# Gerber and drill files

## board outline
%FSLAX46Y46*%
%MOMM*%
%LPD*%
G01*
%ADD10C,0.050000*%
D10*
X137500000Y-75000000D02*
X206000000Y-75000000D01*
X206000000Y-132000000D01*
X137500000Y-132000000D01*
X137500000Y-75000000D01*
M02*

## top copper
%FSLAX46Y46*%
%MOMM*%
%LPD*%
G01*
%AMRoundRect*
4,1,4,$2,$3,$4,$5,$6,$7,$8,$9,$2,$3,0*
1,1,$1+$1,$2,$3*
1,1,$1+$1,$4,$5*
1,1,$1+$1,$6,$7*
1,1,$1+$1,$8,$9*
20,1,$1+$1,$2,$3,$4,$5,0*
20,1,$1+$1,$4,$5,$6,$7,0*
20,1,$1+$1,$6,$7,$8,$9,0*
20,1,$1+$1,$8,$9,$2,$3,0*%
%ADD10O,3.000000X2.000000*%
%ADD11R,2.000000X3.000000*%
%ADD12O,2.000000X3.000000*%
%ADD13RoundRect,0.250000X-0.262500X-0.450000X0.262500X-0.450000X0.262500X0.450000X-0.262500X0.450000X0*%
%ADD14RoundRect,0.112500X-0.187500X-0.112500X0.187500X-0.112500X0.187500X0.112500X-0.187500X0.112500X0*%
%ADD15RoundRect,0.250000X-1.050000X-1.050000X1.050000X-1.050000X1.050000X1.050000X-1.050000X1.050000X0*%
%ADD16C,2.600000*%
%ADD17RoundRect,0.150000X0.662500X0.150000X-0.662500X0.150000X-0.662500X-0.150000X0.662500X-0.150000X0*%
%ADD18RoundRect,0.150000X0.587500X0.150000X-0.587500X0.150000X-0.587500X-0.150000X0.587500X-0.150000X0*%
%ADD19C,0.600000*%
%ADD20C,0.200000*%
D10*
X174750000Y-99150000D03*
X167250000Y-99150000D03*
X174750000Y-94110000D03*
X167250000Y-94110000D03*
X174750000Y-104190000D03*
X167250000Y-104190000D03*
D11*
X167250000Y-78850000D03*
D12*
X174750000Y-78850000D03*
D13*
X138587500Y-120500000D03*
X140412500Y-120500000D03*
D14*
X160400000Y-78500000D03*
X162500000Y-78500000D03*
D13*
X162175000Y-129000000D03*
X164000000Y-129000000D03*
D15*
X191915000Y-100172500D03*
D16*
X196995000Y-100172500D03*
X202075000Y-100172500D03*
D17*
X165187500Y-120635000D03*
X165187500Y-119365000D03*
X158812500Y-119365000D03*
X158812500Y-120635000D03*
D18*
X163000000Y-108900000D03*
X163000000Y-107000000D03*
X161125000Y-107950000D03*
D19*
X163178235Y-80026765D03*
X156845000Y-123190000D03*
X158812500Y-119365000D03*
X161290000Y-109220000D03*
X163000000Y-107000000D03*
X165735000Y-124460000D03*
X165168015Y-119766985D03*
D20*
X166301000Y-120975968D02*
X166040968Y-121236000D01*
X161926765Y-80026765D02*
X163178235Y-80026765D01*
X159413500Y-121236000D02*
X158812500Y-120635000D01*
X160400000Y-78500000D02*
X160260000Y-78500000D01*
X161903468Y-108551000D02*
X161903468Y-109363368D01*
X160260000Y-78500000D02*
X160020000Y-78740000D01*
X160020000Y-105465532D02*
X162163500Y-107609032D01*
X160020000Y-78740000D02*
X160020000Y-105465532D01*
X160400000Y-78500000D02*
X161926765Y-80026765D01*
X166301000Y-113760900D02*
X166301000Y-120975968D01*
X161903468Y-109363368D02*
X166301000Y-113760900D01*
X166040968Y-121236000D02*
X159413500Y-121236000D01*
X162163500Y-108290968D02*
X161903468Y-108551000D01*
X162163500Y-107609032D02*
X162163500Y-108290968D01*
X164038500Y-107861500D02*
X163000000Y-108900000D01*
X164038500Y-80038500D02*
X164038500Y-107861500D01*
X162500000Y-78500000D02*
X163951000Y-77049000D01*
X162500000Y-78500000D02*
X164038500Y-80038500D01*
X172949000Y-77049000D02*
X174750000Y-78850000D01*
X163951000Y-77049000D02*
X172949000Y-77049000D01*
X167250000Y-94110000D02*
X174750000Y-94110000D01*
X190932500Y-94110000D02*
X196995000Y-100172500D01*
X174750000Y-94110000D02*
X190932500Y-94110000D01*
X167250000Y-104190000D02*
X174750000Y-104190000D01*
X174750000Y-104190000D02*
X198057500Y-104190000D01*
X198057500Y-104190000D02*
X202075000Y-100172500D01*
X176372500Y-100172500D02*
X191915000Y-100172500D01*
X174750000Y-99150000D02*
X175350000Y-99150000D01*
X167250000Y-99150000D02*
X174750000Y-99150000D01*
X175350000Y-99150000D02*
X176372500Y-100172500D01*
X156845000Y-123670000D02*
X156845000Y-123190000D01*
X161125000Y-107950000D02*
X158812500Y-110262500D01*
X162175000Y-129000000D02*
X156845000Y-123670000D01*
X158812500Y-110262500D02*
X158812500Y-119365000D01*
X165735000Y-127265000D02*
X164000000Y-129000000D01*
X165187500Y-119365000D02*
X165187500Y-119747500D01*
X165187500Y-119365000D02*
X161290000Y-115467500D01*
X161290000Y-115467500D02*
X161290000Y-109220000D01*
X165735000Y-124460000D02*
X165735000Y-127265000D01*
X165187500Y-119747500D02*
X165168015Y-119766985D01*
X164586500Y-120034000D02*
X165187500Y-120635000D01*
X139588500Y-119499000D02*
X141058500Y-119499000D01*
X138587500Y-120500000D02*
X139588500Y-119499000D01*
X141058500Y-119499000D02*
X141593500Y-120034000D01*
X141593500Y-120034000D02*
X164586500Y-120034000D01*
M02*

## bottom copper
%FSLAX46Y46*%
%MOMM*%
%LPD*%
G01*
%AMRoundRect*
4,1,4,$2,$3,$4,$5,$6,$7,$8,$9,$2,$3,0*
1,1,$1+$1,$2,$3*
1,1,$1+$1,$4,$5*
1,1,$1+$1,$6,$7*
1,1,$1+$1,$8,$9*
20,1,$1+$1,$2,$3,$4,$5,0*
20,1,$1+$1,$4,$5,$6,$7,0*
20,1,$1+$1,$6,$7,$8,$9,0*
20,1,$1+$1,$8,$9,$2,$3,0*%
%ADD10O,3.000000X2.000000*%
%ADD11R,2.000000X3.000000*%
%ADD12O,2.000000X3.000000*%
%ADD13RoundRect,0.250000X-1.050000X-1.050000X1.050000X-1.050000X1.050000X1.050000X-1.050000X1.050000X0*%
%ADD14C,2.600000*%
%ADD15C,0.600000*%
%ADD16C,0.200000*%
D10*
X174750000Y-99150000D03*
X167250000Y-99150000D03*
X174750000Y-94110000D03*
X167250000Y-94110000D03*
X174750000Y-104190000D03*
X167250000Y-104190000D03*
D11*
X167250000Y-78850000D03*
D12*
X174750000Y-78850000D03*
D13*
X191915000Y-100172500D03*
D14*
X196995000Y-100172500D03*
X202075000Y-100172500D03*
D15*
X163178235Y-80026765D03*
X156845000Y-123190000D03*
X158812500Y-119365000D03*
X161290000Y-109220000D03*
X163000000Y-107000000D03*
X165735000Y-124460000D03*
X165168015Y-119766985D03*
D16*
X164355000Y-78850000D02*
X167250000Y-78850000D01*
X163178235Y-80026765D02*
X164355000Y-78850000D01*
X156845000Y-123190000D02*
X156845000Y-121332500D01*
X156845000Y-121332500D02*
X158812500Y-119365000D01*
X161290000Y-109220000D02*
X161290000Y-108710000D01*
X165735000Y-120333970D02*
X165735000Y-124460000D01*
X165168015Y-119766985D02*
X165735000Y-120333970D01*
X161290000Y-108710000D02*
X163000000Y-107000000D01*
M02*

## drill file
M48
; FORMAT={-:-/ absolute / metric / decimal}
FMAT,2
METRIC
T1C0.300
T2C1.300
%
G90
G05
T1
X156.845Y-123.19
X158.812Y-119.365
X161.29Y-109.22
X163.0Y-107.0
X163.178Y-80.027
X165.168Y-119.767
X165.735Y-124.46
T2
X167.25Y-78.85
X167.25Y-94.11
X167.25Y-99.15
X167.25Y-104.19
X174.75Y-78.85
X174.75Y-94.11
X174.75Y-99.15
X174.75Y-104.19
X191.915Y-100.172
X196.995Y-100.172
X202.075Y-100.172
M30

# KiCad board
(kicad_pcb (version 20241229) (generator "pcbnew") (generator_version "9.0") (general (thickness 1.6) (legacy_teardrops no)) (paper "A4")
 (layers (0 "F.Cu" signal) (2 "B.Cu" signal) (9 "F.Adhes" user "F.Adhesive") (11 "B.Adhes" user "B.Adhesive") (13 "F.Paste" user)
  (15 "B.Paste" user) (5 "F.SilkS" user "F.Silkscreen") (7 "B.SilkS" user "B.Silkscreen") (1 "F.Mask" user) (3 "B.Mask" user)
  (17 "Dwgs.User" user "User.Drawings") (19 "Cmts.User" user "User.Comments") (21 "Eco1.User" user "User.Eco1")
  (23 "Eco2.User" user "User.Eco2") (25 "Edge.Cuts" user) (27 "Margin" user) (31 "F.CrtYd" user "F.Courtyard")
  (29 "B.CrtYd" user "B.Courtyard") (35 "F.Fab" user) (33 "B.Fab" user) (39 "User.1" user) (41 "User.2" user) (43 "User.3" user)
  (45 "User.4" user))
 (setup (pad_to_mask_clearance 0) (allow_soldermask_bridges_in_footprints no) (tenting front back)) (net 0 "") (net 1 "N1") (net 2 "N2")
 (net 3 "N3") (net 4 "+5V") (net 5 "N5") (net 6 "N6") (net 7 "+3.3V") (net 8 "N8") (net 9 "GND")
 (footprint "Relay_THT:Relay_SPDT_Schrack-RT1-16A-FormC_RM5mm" (layer "F.Cu") (at 167.25 78.85 -90)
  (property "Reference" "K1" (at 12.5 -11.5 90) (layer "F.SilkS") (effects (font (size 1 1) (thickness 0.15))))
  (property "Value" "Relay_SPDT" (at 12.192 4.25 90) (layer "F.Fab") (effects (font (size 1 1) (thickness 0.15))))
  (pad "11" thru_hole oval (at 20.3 -7.5 90) (size 2 3) (drill 1.3) (layers "*.Cu" "*.Mask") (remove_unused_layers no) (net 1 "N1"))
  (pad "11" thru_hole oval (at 20.3 0 90) (size 2 3) (drill 1.3) (layers "*.Cu" "*.Mask") (remove_unused_layers no) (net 1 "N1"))
  (pad "12" thru_hole oval (at 15.26 -7.5 90) (size 2 3) (drill 1.3) (layers "*.Cu" "*.Mask") (remove_unused_layers no) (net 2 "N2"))
  (pad "12" thru_hole oval (at 15.26 0 90) (size 2 3) (drill 1.3) (layers "*.Cu" "*.Mask") (remove_unused_layers no) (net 2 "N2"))
  (pad "14" thru_hole oval (at 25.34 -7.5 90) (size 2 3) (drill 1.3) (layers "*.Cu" "*.Mask") (remove_unused_layers no) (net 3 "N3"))
  (pad "14" thru_hole oval (at 25.34 0 90) (size 2 3) (drill 1.3) (layers "*.Cu" "*.Mask") (remove_unused_layers no) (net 3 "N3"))
  (pad "A1" thru_hole rect (at 0 0 90) (size 3 2) (drill 1.3) (layers "*.Cu" "*.Mask") (remove_unused_layers no) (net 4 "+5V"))
  (pad "A2" thru_hole oval (at 0 -7.5 90) (size 3 2) (drill 1.3) (layers "*.Cu" "*.Mask") (remove_unused_layers no) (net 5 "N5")))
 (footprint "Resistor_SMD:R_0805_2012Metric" (layer "F.Cu") (at 139.5 120.5)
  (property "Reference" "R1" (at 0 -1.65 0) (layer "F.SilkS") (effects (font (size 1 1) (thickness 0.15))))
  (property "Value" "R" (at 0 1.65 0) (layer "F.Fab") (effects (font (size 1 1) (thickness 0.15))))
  (pad "1" smd roundrect (at -0.9125 0) (size 1.025 1.4) (layers "F.Cu" "F.Mask" "F.Paste") (roundrect_rratio 0.243902) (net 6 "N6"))
  (pad "2" smd roundrect (at 0.9125 0) (size 1.025 1.4) (layers "F.Cu" "F.Mask" "F.Paste") (roundrect_rratio 0.243902) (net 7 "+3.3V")))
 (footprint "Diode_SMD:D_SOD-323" (layer "F.Cu") (at 161.45 78.5)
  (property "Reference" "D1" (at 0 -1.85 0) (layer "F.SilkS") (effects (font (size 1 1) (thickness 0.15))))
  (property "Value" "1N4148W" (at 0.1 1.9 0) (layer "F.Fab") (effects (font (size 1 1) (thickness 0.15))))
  (pad "1" smd roundrect (at -1.05 0) (size 0.6 0.45) (layers "F.Cu" "F.Mask" "F.Paste") (roundrect_rratio 0.25) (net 4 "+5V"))
  (pad "2" smd roundrect (at 1.05 0) (size 0.6 0.45) (layers "F.Cu" "F.Mask" "F.Paste") (roundrect_rratio 0.25) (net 5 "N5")))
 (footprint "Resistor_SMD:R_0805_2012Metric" (layer "F.Cu") (at 163.0875 129)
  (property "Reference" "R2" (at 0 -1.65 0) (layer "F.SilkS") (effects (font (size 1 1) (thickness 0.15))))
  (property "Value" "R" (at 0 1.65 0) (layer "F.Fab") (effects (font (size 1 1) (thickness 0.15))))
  (pad "1" smd roundrect (at -0.9125 0) (size 1.025 1.4) (layers "F.Cu" "F.Mask" "F.Paste") (roundrect_rratio 0.243902) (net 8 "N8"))
  (pad "2" smd roundrect (at 0.9125 0) (size 1.025 1.4) (layers "F.Cu" "F.Mask" "F.Paste") (roundrect_rratio 0.243902) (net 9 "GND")))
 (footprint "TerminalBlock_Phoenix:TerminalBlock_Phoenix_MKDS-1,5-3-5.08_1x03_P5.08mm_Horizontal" (layer "F.Cu") (at 191.915 100.1725)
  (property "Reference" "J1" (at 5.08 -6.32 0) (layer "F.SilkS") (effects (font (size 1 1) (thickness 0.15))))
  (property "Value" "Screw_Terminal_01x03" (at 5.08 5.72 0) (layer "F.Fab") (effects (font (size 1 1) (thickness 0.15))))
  (pad "1" thru_hole roundrect (at 0 0) (size 2.6 2.6) (drill 1.3) (layers "*.Cu" "*.Mask") (remove_unused_layers no)
   (roundrect_rratio 0.096154) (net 1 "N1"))
  (pad "2" thru_hole circle (at 5.08 0) (size 2.6 2.6) (drill 1.3) (layers "*.Cu" "*.Mask") (remove_unused_layers no) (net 2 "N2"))
  (pad "3" thru_hole circle (at 10.16 0) (size 2.6 2.6) (drill 1.3) (layers "*.Cu" "*.Mask") (remove_unused_layers no) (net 3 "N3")))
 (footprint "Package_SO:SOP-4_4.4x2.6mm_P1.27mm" (layer "F.Cu") (at 162 120 180)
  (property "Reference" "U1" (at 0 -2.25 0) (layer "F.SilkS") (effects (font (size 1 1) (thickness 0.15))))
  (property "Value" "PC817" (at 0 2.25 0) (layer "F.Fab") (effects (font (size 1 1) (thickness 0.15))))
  (pad "1" smd roundrect (at -3.1875 -0.635 180) (size 1.625 0.6) (layers "F.Cu" "F.Mask" "F.Paste") (roundrect_rratio 0.25) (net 6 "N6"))
  (pad "2" smd roundrect (at -3.1875 0.635 180) (size 1.625 0.6) (layers "F.Cu" "F.Mask" "F.Paste") (roundrect_rratio 0.25) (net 9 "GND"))
  (pad "3" smd roundrect (at 3.1875 0.635 180) (size 1.625 0.6) (layers "F.Cu" "F.Mask" "F.Paste") (roundrect_rratio 0.25) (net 8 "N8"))
  (pad "4" smd roundrect (at 3.1875 -0.635 180) (size 1.625 0.6) (layers "F.Cu" "F.Mask" "F.Paste") (roundrect_rratio 0.25) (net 4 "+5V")))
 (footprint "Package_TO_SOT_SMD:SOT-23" (layer "F.Cu") (at 162.0625 107.95 180)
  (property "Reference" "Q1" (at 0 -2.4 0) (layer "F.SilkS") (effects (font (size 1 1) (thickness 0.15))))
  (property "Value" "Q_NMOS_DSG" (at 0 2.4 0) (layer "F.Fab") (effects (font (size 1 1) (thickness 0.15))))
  (pad "1" smd roundrect (at -0.9375 -0.95 180) (size 1.475 0.6) (layers "F.Cu" "F.Mask" "F.Paste") (roundrect_rratio 0.25) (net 5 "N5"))
  (pad "2" smd roundrect (at -0.9375 0.95 180) (size 1.475 0.6) (layers "F.Cu" "F.Mask" "F.Paste") (roundrect_rratio 0.25) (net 9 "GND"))
  (pad "3" smd roundrect (at 0.9375 0 180) (size 1.475 0.6) (layers "F.Cu" "F.Mask" "F.Paste") (roundrect_rratio 0.25) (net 8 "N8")))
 (gr_rect (start 137.5 75) (end 206 132) (stroke (width 0.05) (type default)) (fill no) (layer "Edge.Cuts"))
 (segment (start 166.301 120.975968) (end 166.040968 121.236) (width 0.2) (layer "F.Cu") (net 4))
 (segment (start 161.926765 80.026765) (end 163.178235 80.026765) (width 0.2) (layer "F.Cu") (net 4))
 (segment (start 159.4135 121.236) (end 158.8125 120.635) (width 0.2) (layer "F.Cu") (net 4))
 (segment (start 160.4 78.5) (end 160.26 78.5) (width 0.2) (layer "F.Cu") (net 4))
 (segment (start 161.903468 108.551) (end 161.903468 109.363368) (width 0.2) (layer "F.Cu") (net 4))
 (segment (start 160.26 78.5) (end 160.02 78.74) (width 0.2) (layer "F.Cu") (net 4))
 (segment (start 160.02 105.465532) (end 162.1635 107.609032) (width 0.2) (layer "F.Cu") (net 4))
 (segment (start 160.02 78.74) (end 160.02 105.465532) (width 0.2) (layer "F.Cu") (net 4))
 (segment (start 160.4 78.5) (end 161.926765 80.026765) (width 0.2) (layer "F.Cu") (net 4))
 (segment (start 166.301 113.7609) (end 166.301 120.975968) (width 0.2) (layer "F.Cu") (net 4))
 (segment (start 161.903468 109.363368) (end 166.301 113.7609) (width 0.2) (layer "F.Cu") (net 4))
 (segment (start 166.040968 121.236) (end 159.4135 121.236) (width 0.2) (layer "F.Cu") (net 4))
 (segment (start 162.1635 108.290968) (end 161.903468 108.551) (width 0.2) (layer "F.Cu") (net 4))
 (segment (start 162.1635 107.609032) (end 162.1635 108.290968) (width 0.2) (layer "F.Cu") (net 4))
 (via (at 163.178235 80.026765) (size 0.6) (drill 0.3) (layers "F.Cu" "B.Cu") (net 4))
 (segment (start 164.355 78.85) (end 167.25 78.85) (width 0.2) (layer "B.Cu") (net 4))
 (segment (start 163.178235 80.026765) (end 164.355 78.85) (width 0.2) (layer "B.Cu") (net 4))
 (segment (start 164.0385 107.8615) (end 163 108.9) (width 0.2) (layer "F.Cu") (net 5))
 (segment (start 164.0385 80.0385) (end 164.0385 107.8615) (width 0.2) (layer "F.Cu") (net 5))
 (segment (start 162.5 78.5) (end 163.951 77.049) (width 0.2) (layer "F.Cu") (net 5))
 (segment (start 162.5 78.5) (end 164.0385 80.0385) (width 0.2) (layer "F.Cu") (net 5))
 (segment (start 172.949 77.049) (end 174.75 78.85) (width 0.2) (layer "F.Cu") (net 5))
 (segment (start 163.951 77.049) (end 172.949 77.049) (width 0.2) (layer "F.Cu") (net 5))
 (segment (start 167.25 94.11) (end 174.75 94.11) (width 0.2) (layer "F.Cu") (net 2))
 (segment (start 190.9325 94.11) (end 196.995 100.1725) (width 0.2) (layer "F.Cu") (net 2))
 (segment (start 174.75 94.11) (end 190.9325 94.11) (width 0.2) (layer "F.Cu") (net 2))
 (segment (start 167.25 104.19) (end 174.75 104.19) (width 0.2) (layer "F.Cu") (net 3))
 (segment (start 174.75 104.19) (end 198.0575 104.19) (width 0.2) (layer "F.Cu") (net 3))
 (segment (start 198.0575 104.19) (end 202.075 100.1725) (width 0.2) (layer "F.Cu") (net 3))
 (segment (start 176.3725 100.1725) (end 191.915 100.1725) (width 0.2) (layer "F.Cu") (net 1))
 (segment (start 174.75 99.15) (end 175.35 99.15) (width 0.2) (layer "F.Cu") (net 1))
 (segment (start 167.25 99.15) (end 174.75 99.15) (width 0.2) (layer "F.Cu") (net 1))
 (segment (start 175.35 99.15) (end 176.3725 100.1725) (width 0.2) (layer "F.Cu") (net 1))
 (segment (start 156.845 123.67) (end 156.845 123.19) (width 0.2) (layer "F.Cu") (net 8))
 (segment (start 161.125 107.95) (end 158.8125 110.2625) (width 0.2) (layer "F.Cu") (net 8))
 (segment (start 162.175 129) (end 156.845 123.67) (width 0.2) (layer "F.Cu") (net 8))
 (segment (start 158.8125 110.2625) (end 158.8125 119.365) (width 0.2) (layer "F.Cu") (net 8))
 (via (at 156.845 123.19) (size 0.6) (drill 0.3) (layers "F.Cu" "B.Cu") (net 8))
 (via (at 158.8125 119.365) (size 0.6) (drill 0.3) (layers "F.Cu" "B.Cu") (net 8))
 (segment (start 156.845 123.19) (end 156.845 121.3325) (width 0.2) (layer "B.Cu") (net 8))
 (segment (start 156.845 121.3325) (end 158.8125 119.365) (width 0.2) (layer "B.Cu") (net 8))
 (segment (start 165.735 127.265) (end 164 129) (width 0.2) (layer "F.Cu") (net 9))
 (segment (start 165.1875 119.365) (end 165.1875 119.7475) (width 0.2) (layer "F.Cu") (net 9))
 (segment (start 165.1875 119.365) (end 161.29 115.4675) (width 0.2) (layer "F.Cu") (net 9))
 (segment (start 161.29 115.4675) (end 161.29 109.22) (width 0.2) (layer "F.Cu") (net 9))
 (segment (start 165.735 124.46) (end 165.735 127.265) (width 0.2) (layer "F.Cu") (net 9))
 (segment (start 165.1875 119.7475) (end 165.168015 119.766985) (width 0.2) (layer "F.Cu") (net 9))
 (via (at 161.29 109.22) (size 0.6) (drill 0.3) (layers "F.Cu" "B.Cu") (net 9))
 (via (at 163 107) (size 0.6) (drill 0.3) (layers "F.Cu" "B.Cu") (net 9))
 (via (at 165.735 124.46) (size 0.6) (drill 0.3) (layers "F.Cu" "B.Cu") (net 9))
 (via (at 165.168015 119.766985) (size 0.6) (drill 0.3) (layers "F.Cu" "B.Cu") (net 9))
 (segment (start 161.29 109.22) (end 161.29 108.71) (width 0.2) (layer "B.Cu") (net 9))
 (segment (start 165.735 120.33397) (end 165.735 124.46) (width 0.2) (layer "B.Cu") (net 9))
 (segment (start 165.168015 119.766985) (end 165.735 120.33397) (width 0.2) (layer "B.Cu") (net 9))
 (segment (start 161.29 108.71) (end 163 107) (width 0.2) (layer "B.Cu") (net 9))
 (segment (start 164.5865 120.034) (end 165.1875 120.635) (width 0.2) (layer "F.Cu") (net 6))
 (segment (start 139.5885 119.499) (end 141.0585 119.499) (width 0.2) (layer "F.Cu") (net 6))
 (segment (start 138.5875 120.5) (end 139.5885 119.499) (width 0.2) (layer "F.Cu") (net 6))
 (segment (start 141.0585 119.499) (end 141.5935 120.034) (width 0.2) (layer "F.Cu") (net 6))
 (segment (start 141.5935 120.034) (end 164.5865 120.034) (width 0.2) (layer "F.Cu") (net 6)))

